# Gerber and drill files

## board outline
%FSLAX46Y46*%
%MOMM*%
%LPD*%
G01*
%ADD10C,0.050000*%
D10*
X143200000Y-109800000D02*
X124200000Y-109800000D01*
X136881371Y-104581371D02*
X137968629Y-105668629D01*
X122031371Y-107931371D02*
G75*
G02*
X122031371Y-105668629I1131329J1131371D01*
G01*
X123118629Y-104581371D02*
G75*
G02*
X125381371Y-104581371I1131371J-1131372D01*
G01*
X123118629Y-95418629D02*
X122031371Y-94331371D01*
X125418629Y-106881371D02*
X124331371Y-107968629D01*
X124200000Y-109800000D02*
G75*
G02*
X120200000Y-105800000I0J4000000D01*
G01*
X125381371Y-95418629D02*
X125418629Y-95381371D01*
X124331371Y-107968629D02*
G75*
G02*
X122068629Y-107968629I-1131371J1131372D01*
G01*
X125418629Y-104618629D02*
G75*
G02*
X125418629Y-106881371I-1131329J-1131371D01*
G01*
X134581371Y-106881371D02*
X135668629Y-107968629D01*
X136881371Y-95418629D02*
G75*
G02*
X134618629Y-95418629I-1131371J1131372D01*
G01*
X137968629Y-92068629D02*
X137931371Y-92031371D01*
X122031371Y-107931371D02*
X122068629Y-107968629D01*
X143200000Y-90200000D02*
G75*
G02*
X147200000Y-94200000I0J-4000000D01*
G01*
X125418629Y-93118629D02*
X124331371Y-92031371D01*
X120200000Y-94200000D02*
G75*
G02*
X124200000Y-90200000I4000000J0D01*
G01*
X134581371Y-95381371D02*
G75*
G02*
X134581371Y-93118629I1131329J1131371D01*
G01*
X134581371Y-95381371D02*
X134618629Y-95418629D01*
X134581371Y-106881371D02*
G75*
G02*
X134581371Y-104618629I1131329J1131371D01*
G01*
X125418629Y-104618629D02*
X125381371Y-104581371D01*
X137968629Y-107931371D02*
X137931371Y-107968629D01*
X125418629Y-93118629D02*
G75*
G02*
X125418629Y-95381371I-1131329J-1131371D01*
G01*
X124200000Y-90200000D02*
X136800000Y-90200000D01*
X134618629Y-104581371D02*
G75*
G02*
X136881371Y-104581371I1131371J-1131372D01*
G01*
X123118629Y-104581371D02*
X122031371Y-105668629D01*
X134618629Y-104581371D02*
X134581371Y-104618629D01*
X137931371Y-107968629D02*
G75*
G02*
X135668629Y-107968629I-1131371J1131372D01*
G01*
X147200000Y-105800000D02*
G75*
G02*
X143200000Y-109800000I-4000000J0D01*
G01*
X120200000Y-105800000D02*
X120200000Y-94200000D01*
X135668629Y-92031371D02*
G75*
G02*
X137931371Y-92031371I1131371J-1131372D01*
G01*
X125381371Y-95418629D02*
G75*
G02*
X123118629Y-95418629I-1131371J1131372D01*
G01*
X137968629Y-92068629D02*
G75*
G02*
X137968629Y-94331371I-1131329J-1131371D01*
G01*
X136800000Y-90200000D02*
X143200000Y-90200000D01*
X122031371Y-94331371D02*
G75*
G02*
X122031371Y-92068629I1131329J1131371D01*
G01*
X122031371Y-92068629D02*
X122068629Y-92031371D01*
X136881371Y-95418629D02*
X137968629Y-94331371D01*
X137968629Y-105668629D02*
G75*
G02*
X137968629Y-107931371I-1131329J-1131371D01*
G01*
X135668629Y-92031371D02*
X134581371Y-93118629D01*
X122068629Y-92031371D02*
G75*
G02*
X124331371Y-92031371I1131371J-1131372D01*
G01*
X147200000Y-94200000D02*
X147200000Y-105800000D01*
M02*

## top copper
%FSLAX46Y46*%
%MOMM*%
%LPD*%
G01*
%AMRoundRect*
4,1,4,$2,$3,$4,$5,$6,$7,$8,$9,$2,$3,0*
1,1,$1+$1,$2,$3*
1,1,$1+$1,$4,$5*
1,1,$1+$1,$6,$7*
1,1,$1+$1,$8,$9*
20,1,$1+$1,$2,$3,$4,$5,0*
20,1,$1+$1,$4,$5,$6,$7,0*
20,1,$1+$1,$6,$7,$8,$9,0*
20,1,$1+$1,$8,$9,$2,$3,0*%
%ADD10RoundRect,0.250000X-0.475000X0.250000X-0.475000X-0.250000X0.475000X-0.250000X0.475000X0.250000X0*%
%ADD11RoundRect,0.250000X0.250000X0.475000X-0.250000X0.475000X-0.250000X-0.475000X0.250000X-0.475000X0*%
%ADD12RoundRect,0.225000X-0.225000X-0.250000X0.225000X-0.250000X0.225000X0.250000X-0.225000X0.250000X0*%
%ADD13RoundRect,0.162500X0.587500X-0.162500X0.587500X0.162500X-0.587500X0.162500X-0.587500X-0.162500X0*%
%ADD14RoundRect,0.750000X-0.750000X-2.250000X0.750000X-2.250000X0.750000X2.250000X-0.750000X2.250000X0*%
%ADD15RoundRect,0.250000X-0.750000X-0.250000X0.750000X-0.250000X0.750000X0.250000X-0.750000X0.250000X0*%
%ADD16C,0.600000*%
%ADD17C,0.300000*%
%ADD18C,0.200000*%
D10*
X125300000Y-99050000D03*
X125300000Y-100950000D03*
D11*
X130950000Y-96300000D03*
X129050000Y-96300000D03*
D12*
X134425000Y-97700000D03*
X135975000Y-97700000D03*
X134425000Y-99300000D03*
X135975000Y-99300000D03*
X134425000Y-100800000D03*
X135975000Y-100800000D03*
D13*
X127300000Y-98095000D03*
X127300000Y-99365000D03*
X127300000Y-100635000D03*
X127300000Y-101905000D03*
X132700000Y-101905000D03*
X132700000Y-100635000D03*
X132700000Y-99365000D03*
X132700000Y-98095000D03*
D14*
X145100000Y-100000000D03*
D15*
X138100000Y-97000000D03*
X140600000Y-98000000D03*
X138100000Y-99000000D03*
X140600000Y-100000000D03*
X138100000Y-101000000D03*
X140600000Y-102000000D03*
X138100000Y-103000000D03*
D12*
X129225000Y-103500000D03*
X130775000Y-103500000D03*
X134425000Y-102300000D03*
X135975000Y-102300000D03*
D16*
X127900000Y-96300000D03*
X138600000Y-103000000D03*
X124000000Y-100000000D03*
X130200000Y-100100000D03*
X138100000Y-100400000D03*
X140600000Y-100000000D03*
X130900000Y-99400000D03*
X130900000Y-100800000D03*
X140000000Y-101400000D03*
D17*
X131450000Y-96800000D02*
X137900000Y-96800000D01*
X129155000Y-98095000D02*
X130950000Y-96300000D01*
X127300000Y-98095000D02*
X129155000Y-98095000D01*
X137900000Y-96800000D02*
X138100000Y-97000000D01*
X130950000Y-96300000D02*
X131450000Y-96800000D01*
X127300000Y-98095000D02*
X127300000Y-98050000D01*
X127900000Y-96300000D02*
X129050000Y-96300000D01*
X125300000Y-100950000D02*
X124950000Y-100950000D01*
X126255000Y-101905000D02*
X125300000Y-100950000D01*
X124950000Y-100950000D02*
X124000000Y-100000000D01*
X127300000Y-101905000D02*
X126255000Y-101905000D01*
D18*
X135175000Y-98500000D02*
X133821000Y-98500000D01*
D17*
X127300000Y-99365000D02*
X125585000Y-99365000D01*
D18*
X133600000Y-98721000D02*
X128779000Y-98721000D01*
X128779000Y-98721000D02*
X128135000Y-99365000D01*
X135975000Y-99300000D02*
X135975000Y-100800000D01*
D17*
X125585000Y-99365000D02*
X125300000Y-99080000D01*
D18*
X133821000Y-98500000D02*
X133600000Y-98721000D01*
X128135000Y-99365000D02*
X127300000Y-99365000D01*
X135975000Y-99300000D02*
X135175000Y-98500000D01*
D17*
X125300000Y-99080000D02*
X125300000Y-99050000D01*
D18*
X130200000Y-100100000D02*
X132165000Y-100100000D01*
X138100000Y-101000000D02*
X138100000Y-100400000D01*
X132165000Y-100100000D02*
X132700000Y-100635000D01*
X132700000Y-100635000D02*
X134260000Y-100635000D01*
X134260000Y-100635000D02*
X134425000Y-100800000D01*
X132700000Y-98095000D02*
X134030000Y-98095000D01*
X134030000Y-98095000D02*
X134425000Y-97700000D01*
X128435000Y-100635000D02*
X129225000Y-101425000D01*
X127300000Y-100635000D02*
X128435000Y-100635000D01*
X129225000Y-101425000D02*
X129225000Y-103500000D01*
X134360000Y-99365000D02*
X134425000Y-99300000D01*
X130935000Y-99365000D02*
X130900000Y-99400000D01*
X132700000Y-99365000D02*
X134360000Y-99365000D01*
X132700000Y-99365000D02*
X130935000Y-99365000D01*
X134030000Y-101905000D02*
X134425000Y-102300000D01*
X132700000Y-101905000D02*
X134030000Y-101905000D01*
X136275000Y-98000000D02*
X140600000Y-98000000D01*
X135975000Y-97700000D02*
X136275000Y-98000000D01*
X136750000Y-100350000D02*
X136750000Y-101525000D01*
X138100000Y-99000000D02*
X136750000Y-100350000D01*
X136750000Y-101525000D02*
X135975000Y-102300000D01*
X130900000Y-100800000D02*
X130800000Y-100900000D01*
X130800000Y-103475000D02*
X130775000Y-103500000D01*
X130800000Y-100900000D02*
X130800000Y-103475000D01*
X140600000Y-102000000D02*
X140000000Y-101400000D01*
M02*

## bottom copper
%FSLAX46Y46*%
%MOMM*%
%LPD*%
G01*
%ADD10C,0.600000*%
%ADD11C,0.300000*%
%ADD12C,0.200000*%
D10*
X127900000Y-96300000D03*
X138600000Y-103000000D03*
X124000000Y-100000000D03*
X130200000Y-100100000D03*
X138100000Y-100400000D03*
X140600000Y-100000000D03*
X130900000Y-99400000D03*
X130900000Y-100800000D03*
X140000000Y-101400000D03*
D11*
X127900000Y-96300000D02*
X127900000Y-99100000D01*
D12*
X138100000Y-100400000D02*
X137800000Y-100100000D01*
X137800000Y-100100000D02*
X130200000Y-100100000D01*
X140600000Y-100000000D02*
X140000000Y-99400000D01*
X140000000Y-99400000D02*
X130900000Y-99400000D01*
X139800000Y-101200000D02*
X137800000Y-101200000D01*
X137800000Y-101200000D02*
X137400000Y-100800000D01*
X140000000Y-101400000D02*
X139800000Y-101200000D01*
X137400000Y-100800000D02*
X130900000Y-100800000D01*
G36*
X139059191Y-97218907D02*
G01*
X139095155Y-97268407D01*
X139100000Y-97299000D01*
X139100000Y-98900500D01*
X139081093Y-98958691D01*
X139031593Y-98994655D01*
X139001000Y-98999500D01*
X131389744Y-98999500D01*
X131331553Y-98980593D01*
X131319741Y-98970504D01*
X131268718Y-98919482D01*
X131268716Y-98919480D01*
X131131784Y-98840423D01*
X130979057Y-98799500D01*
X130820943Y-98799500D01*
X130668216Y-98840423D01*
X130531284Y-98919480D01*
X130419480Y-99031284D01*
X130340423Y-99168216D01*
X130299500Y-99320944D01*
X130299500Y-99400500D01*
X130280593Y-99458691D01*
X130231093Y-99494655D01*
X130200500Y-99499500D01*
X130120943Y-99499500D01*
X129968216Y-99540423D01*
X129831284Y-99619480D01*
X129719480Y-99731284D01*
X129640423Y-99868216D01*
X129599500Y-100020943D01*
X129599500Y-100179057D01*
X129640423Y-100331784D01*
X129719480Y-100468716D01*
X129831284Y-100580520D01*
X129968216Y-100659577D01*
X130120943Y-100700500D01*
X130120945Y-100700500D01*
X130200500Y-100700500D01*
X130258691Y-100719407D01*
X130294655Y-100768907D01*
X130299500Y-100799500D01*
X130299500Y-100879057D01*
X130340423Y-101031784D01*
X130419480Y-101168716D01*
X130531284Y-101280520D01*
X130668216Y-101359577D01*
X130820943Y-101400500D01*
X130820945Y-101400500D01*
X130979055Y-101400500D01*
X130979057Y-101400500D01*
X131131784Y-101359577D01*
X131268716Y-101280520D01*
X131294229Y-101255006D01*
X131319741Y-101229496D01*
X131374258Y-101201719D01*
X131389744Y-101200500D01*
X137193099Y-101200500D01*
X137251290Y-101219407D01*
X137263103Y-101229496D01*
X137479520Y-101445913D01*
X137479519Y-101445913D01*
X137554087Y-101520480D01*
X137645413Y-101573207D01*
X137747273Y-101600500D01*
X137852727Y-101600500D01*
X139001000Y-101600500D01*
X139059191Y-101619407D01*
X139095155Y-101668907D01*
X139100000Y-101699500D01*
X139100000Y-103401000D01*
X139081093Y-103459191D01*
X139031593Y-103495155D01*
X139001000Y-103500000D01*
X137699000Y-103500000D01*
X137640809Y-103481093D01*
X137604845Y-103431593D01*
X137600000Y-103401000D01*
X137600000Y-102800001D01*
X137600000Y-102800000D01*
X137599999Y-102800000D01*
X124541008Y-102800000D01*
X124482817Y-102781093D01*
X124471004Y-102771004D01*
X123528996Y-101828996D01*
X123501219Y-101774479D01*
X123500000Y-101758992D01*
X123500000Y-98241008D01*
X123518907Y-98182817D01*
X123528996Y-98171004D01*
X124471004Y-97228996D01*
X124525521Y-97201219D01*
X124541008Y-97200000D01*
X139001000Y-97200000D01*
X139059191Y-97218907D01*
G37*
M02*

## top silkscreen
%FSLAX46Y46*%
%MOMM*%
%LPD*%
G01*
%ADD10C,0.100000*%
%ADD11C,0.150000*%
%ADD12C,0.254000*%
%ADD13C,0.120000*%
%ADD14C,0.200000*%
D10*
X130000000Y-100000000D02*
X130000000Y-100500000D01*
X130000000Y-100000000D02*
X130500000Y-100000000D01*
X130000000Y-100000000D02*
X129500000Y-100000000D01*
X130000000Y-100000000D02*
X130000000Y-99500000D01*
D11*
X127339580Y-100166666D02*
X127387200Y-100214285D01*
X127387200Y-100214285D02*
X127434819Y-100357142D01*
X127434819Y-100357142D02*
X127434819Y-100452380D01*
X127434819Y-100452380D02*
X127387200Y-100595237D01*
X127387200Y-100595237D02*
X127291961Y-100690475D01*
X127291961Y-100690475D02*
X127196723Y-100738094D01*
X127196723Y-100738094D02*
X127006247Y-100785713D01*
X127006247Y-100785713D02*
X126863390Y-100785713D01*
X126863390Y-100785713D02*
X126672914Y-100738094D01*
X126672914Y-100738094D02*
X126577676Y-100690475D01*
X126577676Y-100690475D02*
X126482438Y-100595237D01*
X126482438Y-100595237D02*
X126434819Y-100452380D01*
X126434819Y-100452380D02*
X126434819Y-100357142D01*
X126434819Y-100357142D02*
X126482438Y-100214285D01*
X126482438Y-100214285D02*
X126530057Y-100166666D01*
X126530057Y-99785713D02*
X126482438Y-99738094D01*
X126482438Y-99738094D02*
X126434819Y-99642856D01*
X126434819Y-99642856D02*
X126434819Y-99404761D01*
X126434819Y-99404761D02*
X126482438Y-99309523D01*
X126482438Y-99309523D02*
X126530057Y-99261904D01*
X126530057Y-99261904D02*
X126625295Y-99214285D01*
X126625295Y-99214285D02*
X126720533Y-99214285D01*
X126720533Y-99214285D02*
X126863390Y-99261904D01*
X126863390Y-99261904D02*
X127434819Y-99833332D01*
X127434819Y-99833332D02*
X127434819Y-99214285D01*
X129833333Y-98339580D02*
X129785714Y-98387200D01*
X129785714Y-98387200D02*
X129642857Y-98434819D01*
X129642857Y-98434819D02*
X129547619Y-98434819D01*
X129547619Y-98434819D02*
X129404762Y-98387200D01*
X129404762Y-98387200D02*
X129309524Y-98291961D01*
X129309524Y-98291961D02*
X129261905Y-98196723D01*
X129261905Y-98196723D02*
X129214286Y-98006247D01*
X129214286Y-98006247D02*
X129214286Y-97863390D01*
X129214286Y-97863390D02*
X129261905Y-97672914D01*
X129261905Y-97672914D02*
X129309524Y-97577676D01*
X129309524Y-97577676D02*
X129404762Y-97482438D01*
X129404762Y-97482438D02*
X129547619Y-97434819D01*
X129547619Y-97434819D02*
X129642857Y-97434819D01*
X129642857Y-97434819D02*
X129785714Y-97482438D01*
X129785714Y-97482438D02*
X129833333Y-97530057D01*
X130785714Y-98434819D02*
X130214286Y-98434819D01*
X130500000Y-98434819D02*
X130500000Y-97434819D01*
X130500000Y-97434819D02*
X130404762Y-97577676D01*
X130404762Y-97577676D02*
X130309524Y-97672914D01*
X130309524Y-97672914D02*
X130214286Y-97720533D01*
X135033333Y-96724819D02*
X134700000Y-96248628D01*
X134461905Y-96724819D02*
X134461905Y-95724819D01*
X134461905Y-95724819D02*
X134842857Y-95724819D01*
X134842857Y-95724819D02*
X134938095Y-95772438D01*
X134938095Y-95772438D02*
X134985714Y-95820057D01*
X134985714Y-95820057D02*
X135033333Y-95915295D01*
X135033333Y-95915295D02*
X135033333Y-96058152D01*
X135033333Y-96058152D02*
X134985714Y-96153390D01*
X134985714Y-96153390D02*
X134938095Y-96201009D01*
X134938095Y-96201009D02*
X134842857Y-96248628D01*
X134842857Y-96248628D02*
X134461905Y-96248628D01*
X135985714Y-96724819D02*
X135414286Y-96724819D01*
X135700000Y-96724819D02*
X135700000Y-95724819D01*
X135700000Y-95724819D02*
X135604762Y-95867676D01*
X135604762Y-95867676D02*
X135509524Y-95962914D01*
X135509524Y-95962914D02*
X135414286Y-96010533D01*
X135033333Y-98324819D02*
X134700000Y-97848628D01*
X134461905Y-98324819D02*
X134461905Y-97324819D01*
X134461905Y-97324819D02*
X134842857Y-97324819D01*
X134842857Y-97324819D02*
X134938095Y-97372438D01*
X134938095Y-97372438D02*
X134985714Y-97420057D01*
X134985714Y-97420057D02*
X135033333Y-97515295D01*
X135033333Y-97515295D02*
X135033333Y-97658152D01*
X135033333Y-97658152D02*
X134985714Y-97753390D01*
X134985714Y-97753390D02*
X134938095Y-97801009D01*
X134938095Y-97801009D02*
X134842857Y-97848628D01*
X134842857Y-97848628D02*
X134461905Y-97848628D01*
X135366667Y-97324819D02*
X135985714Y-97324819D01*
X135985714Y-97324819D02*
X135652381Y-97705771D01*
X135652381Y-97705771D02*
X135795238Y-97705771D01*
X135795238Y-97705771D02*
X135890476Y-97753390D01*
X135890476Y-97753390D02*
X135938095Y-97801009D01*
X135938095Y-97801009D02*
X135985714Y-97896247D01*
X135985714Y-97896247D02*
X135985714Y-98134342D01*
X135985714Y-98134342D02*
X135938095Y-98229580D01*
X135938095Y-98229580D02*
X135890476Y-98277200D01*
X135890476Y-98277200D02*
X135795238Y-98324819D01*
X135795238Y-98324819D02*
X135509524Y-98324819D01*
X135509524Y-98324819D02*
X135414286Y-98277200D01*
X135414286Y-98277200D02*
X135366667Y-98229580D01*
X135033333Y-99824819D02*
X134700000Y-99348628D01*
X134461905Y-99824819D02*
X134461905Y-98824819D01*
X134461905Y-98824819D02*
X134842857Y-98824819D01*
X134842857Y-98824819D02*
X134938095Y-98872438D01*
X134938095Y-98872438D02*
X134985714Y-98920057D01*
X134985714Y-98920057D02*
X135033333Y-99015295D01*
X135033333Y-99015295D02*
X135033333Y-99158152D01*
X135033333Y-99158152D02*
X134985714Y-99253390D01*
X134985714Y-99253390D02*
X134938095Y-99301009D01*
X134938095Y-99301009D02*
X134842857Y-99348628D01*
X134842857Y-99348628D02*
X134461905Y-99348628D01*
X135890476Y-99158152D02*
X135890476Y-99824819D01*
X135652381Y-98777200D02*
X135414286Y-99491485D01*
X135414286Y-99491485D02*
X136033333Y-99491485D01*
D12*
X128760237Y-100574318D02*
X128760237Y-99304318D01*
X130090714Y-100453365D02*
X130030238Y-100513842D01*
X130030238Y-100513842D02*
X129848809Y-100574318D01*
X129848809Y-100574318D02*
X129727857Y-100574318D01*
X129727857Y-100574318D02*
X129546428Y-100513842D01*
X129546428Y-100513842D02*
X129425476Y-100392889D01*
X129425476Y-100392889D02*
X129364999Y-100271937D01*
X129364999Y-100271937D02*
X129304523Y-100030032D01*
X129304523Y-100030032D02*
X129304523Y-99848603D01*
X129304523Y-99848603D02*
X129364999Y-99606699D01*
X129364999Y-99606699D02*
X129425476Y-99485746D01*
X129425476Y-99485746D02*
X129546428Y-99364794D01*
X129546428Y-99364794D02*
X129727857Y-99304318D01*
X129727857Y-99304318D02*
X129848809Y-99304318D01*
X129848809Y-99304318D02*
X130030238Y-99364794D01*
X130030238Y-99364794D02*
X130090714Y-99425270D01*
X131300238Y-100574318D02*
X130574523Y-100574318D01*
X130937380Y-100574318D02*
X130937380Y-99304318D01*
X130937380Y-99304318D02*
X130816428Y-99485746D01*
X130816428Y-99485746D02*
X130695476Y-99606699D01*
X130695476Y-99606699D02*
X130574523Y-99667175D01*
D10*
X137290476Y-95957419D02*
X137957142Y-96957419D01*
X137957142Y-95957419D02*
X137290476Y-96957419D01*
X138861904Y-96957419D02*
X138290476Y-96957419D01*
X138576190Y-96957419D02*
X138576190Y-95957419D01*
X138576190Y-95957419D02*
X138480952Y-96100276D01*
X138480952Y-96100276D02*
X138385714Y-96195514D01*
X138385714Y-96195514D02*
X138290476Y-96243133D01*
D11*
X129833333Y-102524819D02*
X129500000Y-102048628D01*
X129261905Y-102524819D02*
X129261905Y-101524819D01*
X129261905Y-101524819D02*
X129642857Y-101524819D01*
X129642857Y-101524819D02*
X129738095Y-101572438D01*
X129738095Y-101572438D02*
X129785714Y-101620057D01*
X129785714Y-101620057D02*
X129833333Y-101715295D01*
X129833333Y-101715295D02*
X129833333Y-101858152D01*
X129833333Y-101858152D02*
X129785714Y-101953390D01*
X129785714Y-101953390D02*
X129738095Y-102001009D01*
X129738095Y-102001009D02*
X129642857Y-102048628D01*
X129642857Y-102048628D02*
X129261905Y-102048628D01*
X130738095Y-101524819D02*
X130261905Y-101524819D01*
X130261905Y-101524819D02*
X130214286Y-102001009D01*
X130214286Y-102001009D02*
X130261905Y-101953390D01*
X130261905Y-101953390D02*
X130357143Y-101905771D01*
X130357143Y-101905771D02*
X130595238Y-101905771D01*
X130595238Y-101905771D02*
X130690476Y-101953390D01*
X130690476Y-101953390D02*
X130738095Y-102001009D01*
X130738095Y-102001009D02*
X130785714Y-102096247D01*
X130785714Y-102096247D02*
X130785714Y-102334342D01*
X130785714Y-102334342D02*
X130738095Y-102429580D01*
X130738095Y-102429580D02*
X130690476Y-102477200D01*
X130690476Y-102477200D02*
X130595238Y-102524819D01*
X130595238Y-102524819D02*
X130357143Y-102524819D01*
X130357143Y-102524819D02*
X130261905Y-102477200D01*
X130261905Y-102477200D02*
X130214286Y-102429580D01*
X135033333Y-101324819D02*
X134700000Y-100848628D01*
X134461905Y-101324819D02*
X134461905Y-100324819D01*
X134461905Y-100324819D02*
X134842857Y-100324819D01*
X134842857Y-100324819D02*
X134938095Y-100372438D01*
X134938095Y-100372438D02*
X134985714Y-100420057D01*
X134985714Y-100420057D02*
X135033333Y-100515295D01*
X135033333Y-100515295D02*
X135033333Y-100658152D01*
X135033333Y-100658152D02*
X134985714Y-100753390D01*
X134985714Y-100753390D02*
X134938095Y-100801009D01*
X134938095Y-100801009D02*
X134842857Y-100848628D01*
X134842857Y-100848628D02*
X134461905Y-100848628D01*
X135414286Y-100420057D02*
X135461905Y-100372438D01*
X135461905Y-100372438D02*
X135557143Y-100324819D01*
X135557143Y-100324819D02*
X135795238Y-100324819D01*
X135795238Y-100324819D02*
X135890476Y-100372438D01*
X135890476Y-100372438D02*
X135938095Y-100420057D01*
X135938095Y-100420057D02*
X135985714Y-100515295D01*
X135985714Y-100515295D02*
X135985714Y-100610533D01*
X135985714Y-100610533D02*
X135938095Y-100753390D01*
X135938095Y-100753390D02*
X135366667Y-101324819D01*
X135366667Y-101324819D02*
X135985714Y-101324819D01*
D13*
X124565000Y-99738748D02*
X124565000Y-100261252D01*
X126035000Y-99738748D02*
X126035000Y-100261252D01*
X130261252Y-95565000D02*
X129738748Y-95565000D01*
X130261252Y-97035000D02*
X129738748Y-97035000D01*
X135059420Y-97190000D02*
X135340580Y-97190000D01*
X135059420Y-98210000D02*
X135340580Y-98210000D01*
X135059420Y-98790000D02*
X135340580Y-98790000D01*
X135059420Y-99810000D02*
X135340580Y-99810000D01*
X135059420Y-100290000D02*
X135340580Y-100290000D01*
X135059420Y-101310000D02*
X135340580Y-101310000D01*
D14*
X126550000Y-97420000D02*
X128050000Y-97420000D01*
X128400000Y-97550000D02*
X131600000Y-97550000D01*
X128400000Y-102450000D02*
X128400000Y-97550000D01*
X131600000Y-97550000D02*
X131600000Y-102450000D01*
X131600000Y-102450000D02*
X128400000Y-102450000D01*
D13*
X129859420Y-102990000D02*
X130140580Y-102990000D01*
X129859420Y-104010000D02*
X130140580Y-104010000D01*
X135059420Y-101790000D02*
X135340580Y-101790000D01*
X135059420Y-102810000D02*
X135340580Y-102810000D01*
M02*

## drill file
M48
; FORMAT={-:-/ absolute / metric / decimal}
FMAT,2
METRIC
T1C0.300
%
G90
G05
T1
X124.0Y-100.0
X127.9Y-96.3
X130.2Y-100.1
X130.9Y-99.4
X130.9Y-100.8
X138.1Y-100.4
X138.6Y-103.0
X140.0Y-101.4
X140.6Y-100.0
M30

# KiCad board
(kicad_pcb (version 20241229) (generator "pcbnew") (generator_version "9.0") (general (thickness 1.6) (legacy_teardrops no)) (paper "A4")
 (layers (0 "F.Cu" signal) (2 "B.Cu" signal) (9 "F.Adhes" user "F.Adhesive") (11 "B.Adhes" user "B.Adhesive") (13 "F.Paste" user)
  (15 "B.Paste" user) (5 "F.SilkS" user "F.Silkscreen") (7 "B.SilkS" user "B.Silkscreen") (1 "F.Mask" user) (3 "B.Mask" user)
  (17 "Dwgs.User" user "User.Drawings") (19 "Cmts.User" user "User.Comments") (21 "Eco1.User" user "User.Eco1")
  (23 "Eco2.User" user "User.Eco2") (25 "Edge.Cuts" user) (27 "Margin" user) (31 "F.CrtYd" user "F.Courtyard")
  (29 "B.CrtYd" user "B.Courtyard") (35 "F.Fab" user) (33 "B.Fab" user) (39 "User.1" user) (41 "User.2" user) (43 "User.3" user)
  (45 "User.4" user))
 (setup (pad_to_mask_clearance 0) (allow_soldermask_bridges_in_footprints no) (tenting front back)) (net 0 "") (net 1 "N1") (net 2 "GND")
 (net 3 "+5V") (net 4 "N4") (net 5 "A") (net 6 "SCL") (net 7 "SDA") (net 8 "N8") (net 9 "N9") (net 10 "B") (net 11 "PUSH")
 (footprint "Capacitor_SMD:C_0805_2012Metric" (layer "F.Cu") (at 125.3 100 -90)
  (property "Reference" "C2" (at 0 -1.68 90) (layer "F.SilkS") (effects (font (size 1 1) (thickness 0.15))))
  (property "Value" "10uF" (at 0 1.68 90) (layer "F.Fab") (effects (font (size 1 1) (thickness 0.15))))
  (fp_line (start -0.261252 0.735) (end 0.261252 0.735) (stroke (width 0.12) (type solid)) (layer "F.SilkS"))
  (fp_line (start -0.261252 -0.735) (end 0.261252 -0.735) (stroke (width 0.12) (type solid)) (layer "F.SilkS"))
  (pad "1" smd roundrect (at -0.95 0 270) (size 1 1.45) (layers "F.Cu" "F.Mask" "F.Paste") (roundrect_rratio 0.25) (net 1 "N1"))
  (pad "2" smd roundrect (at 0.95 0 270) (size 1 1.45) (layers "F.Cu" "F.Mask" "F.Paste") (roundrect_rratio 0.25) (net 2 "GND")))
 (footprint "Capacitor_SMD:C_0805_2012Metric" (layer "F.Cu") (at 130 96.3 180)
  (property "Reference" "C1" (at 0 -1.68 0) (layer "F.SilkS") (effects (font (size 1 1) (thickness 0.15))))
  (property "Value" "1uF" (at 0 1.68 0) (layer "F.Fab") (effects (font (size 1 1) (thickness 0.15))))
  (fp_line (start -0.261252 0.735) (end 0.261252 0.735) (stroke (width 0.12) (type solid)) (layer "F.SilkS"))
  (fp_line (start -0.261252 -0.735) (end 0.261252 -0.735) (stroke (width 0.12) (type solid)) (layer "F.SilkS"))
  (pad "1" smd roundrect (at -0.95 0 180) (size 1 1.45) (layers "F.Cu" "F.Mask" "F.Paste") (roundrect_rratio 0.25) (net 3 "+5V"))
  (pad "2" smd roundrect (at 0.95 0 180) (size 1 1.45) (layers "F.Cu" "F.Mask" "F.Paste") (roundrect_rratio 0.25) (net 2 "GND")))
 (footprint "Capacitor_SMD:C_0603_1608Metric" (layer "F.Cu") (at 135.2 97.7)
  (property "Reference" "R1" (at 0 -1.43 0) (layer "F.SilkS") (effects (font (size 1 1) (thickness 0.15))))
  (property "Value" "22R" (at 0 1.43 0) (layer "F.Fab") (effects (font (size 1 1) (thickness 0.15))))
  (fp_line (start -0.14058 -0.51) (end 0.14058 -0.51) (stroke (width 0.12) (type solid)) (layer "F.SilkS"))
  (fp_line (start -0.14058 0.51) (end 0.14058 0.51) (stroke (width 0.12) (type solid)) (layer "F.SilkS"))
  (pad "1" smd roundrect (at -0.775 0) (size 0.9 0.95) (layers "F.Cu" "F.Mask" "F.Paste") (roundrect_rratio 0.25) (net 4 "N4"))
  (pad "2" smd roundrect (at 0.775 0) (size 0.9 0.95) (layers "F.Cu" "F.Mask" "F.Paste") (roundrect_rratio 0.25) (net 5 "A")))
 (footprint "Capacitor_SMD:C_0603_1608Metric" (layer "F.Cu") (at 135.2 99.3)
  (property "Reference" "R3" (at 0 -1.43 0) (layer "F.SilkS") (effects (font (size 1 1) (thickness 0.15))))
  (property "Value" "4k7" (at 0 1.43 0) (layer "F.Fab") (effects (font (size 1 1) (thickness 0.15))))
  (fp_line (start -0.14058 -0.51) (end 0.14058 -0.51) (stroke (width 0.12) (type solid)) (layer "F.SilkS"))
  (fp_line (start -0.14058 0.51) (end 0.14058 0.51) (stroke (width 0.12) (type solid)) (layer "F.SilkS"))
  (pad "1" smd roundrect (at -0.775 0) (size 0.9 0.95) (layers "F.Cu" "F.Mask" "F.Paste") (roundrect_rratio 0.25) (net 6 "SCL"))
  (pad "2" smd roundrect (at 0.775 0) (size 0.9 0.95) (layers "F.Cu" "F.Mask" "F.Paste") (roundrect_rratio 0.25) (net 1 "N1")))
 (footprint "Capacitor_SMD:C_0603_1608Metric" (layer "F.Cu") (at 135.2 100.8)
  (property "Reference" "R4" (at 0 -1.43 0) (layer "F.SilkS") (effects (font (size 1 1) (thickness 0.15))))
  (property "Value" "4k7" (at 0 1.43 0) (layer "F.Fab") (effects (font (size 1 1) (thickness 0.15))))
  (fp_line (start -0.14058 -0.51) (end 0.14058 -0.51) (stroke (width 0.12) (type solid)) (layer "F.SilkS"))
  (fp_line (start -0.14058 0.51) (end 0.14058 0.51) (stroke (width 0.12) (type solid)) (layer "F.SilkS"))
  (pad "1" smd roundrect (at -0.775 0) (size 0.9 0.95) (layers "F.Cu" "F.Mask" "F.Paste") (roundrect_rratio 0.25) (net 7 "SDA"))
  (pad "2" smd roundrect (at 0.775 0) (size 0.9 0.95) (layers "F.Cu" "F.Mask" "F.Paste") (roundrect_rratio 0.25) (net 1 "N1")))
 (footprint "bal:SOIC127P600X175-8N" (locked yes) (layer "F.Cu") (at 130 100)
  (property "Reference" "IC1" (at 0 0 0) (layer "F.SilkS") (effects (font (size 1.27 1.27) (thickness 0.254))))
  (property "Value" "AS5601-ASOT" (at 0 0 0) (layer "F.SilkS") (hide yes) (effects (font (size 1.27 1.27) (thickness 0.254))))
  (fp_line (start -3.45 -2.58) (end -1.95 -2.58) (stroke (width 0.2) (type solid)) (layer "F.SilkS"))
  (fp_line (start -1.6 -2.45) (end 1.6 -2.45) (stroke (width 0.2) (type solid)) (layer "F.SilkS"))
  (fp_line (start -1.6 2.45) (end -1.6 -2.45) (stroke (width 0.2) (type solid)) (layer "F.SilkS"))
  (fp_line (start 1.6 -2.45) (end 1.6 2.45) (stroke (width 0.2) (type solid)) (layer "F.SilkS"))
  (fp_line (start 1.6 2.45) (end -1.6 2.45) (stroke (width 0.2) (type solid)) (layer "F.SilkS"))
  (pad "1" smd roundrect (at -2.7 -1.905 90) (size 0.65 1.5) (layers "F.Cu" "F.Mask" "F.Paste") (roundrect_rratio 0.25) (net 3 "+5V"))
  (pad "2" smd roundrect (at -2.7 -0.635 90) (size 0.65 1.5) (layers "F.Cu" "F.Mask" "F.Paste") (roundrect_rratio 0.25) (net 1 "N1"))
  (pad "3" smd roundrect (at -2.7 0.635 90) (size 0.65 1.5) (layers "F.Cu" "F.Mask" "F.Paste") (roundrect_rratio 0.25) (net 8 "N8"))
  (pad "4" smd roundrect (at -2.7 1.905 90) (size 0.65 1.5) (layers "F.Cu" "F.Mask" "F.Paste") (roundrect_rratio 0.25) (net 2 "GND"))
  (pad "5" smd roundrect (at 2.7 1.905 90) (size 0.65 1.5) (layers "F.Cu" "F.Mask" "F.Paste") (roundrect_rratio 0.25) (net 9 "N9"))
  (pad "6" smd roundrect (at 2.7 0.635 90) (size 0.65 1.5) (layers "F.Cu" "F.Mask" "F.Paste") (roundrect_rratio 0.25) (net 7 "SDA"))
  (pad "7" smd roundrect (at 2.7 -0.635 90) (size 0.65 1.5) (layers "F.Cu" "F.Mask" "F.Paste") (roundrect_rratio 0.25) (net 6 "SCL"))
  (pad "8" smd roundrect (at 2.7 -1.905 90) (size 0.65 1.5) (layers "F.Cu" "F.Mask" "F.Paste") (roundrect_rratio 0.25) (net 4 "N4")))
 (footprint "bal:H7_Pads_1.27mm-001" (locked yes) (layer "F.Cu") (at 138.1 97)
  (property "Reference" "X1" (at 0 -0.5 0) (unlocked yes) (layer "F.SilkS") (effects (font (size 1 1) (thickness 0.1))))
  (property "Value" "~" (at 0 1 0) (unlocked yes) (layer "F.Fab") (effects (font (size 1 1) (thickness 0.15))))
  (pad "" smd roundrect (at 7 3) (size 3 6) (layers "F.Cu" "F.Mask" "F.Paste") (roundrect_rratio 0.25) (thermal_bridge_angle 45))
  (pad "1" smd roundrect (at 0 0) (size 2 1) (layers "F.Cu" "F.Mask" "F.Paste") (roundrect_rratio 0.25) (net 3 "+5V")
   (thermal_bridge_angle 45))
  (pad "2" smd roundrect (at 2.5 1) (size 2 1) (layers "F.Cu" "F.Mask" "F.Paste") (roundrect_rratio 0.25) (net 5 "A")
   (thermal_bridge_angle 45))
  (pad "3" smd roundrect (at 0 2) (size 2 1) (layers "F.Cu" "F.Mask" "F.Paste") (roundrect_rratio 0.25) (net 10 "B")
   (thermal_bridge_angle 45))
  (pad "4" smd roundrect (at 2.5 3) (size 2 1) (layers "F.Cu" "F.Mask" "F.Paste") (roundrect_rratio 0.25) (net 6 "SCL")
   (thermal_bridge_angle 45))
  (pad "5" smd roundrect (at 0 4) (size 2 1) (layers "F.Cu" "F.Mask" "F.Paste") (roundrect_rratio 0.25) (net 7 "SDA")
   (thermal_bridge_angle 45))
  (pad "6" smd roundrect (at 2.5 5) (size 2 1) (layers "F.Cu" "F.Mask" "F.Paste") (roundrect_rratio 0.25) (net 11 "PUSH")
   (thermal_bridge_angle 45))
  (pad "7" smd roundrect (at 0 6) (size 2 1) (layers "F.Cu" "F.Mask" "F.Paste") (roundrect_rratio 0.25) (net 2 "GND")
   (thermal_bridge_angle 45)))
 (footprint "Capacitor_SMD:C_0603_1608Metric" (layer "F.Cu") (at 130 103.5)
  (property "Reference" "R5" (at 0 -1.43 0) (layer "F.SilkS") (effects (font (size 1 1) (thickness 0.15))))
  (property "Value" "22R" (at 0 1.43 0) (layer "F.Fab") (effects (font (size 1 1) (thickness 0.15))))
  (fp_line (start -0.14058 -0.51) (end 0.14058 -0.51) (stroke (width 0.12) (type solid)) (layer "F.SilkS"))
  (fp_line (start -0.14058 0.51) (end 0.14058 0.51) (stroke (width 0.12) (type solid)) (layer "F.SilkS"))
  (pad "1" smd roundrect (at -0.775 0) (size 0.9 0.95) (layers "F.Cu" "F.Mask" "F.Paste") (roundrect_rratio 0.25) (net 8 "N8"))
  (pad "2" smd roundrect (at 0.775 0) (size 0.9 0.95) (layers "F.Cu" "F.Mask" "F.Paste") (roundrect_rratio 0.25) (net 11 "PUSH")))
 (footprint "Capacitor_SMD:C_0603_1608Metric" (layer "F.Cu") (at 135.2 102.3)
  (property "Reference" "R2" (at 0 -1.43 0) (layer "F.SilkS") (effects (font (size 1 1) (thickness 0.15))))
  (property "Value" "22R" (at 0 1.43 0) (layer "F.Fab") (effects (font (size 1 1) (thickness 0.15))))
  (fp_line (start -0.14058 -0.51) (end 0.14058 -0.51) (stroke (width 0.12) (type solid)) (layer "F.SilkS"))
  (fp_line (start -0.14058 0.51) (end 0.14058 0.51) (stroke (width 0.12) (type solid)) (layer "F.SilkS"))
  (pad "1" smd roundrect (at -0.775 0) (size 0.9 0.95) (layers "F.Cu" "F.Mask" "F.Paste") (roundrect_rratio 0.25) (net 9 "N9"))
  (pad "2" smd roundrect (at 0.775 0) (size 0.9 0.95) (layers "F.Cu" "F.Mask" "F.Paste") (roundrect_rratio 0.25) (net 10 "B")))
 (gr_line (start 130 100) (end 130 100.5) (stroke (width 0.1) (type default)) (layer "F.SilkS"))
 (gr_line (start 130 100) (end 130.5 100) (stroke (width 0.1) (type default)) (layer "F.SilkS"))
 (gr_line (start 130 100) (end 129.5 100) (stroke (width 0.1) (type default)) (layer "F.SilkS"))
 (gr_line (start 130 100) (end 130 99.5) (stroke (width 0.1) (type default)) (layer "F.SilkS"))
 (gr_line (start 143.2 109.8) (end 124.2 109.8) (stroke (width 0.05) (type default)) (layer "Edge.Cuts"))
 (gr_line (start 136.881371 104.581371) (end 137.968629 105.668629) (stroke (width 0.05) (type default)) (layer "Edge.Cuts"))
 (gr_arc (start 122.031371 107.931371) (mid 121.562729 106.8) (end 122.031371 105.668629) (stroke (width 0.05) (type default))
  (layer "Edge.Cuts"))
 (gr_arc (start 123.118629 104.581371) (mid 124.25 104.112742) (end 125.381371 104.581371) (stroke (width 0.05) (type default))
  (layer "Edge.Cuts"))
 (gr_line (start 123.118629 95.418629) (end 122.031371 94.331371) (stroke (width 0.05) (type default)) (layer "Edge.Cuts"))
 (gr_line (start 125.418629 106.881371) (end 124.331371 107.968629) (stroke (width 0.05) (type default)) (layer "Edge.Cuts"))
 (gr_arc (start 124.2 109.8) (mid 121.371573 108.628427) (end 120.2 105.8) (stroke (width 0.05) (type default)) (layer "Edge.Cuts"))
 (gr_line (start 125.381371 95.418629) (end 125.418629 95.381371) (stroke (width 0.05) (type default)) (layer "Edge.Cuts"))
 (gr_arc (start 124.331371 107.968629) (mid 123.2 108.437258) (end 122.068629 107.968629) (stroke (width 0.05) (type default))
  (layer "Edge.Cuts"))
 (gr_arc (start 125.418629 104.618629) (mid 125.887258 105.75) (end 125.418629 106.881371) (stroke (width 0.05) (type default))
  (layer "Edge.Cuts"))
 (gr_line (start 134.581371 106.881371) (end 135.668629 107.968629) (stroke (width 0.05) (type default)) (layer "Edge.Cuts"))
 (gr_arc (start 136.881371 95.418629) (mid 135.75 95.887258) (end 134.618629 95.418629) (stroke (width 0.05) (type default))
  (layer "Edge.Cuts"))
 (gr_line (start 137.968629 92.068629) (end 137.931371 92.031371) (stroke (width 0.05) (type default)) (layer "Edge.Cuts"))
 (gr_line (start 122.031371 107.931371) (end 122.068629 107.968629) (stroke (width 0.05) (type default)) (layer "Edge.Cuts"))
 (gr_arc (start 143.2 90.2) (mid 146.028427 91.371573) (end 147.2 94.2) (stroke (width 0.05) (type default)) (layer "Edge.Cuts"))
 (gr_line (start 125.418629 93.118629) (end 124.331371 92.031371) (stroke (width 0.05) (type default)) (layer "Edge.Cuts"))
 (gr_arc (start 120.2 94.2) (mid 121.371573 91.371573) (end 124.2 90.2) (stroke (width 0.05) (type default)) (layer "Edge.Cuts"))
 (gr_arc (start 134.581371 95.381371) (mid 134.112729 94.25) (end 134.581371 93.118629) (stroke (width 0.05) (type default))
  (layer "Edge.Cuts"))
 (gr_line (start 134.581371 95.381371) (end 134.618629 95.418629) (stroke (width 0.05) (type default)) (layer "Edge.Cuts"))
 (gr_arc (start 134.581371 106.881371) (mid 134.112729 105.75) (end 134.581371 104.618629) (stroke (width 0.05) (type default))
  (layer "Edge.Cuts"))
 (gr_line (start 125.418629 104.618629) (end 125.381371 104.581371) (stroke (width 0.05) (type default)) (layer "Edge.Cuts"))
 (gr_line (start 137.968629 107.931371) (end 137.931371 107.968629) (stroke (width 0.05) (type default)) (layer "Edge.Cuts"))
 (gr_arc (start 125.418629 93.118629) (mid 125.887258 94.25) (end 125.418629 95.381371) (stroke (width 0.05) (type default))
  (layer "Edge.Cuts"))
 (gr_line (start 124.2 90.2) (end 136.8 90.2) (stroke (width 0.05) (type default)) (layer "Edge.Cuts"))
 (gr_arc (start 134.618629 104.581371) (mid 135.75 104.112742) (end 136.881371 104.581371) (stroke (width 0.05) (type default))
  (layer "Edge.Cuts"))
 (gr_line (start 123.118629 104.581371) (end 122.031371 105.668629) (stroke (width 0.05) (type default)) (layer "Edge.Cuts"))
 (gr_line (start 134.618629 104.581371) (end 134.581371 104.618629) (stroke (width 0.05) (type default)) (layer "Edge.Cuts"))
 (gr_arc (start 137.931371 107.968629) (mid 136.8 108.437258) (end 135.668629 107.968629) (stroke (width 0.05) (type default))
  (layer "Edge.Cuts"))
 (gr_arc (start 147.2 105.8) (mid 146.028427 108.628427) (end 143.2 109.8) (stroke (width 0.05) (type default)) (layer "Edge.Cuts"))
 (gr_line (start 120.2 105.8) (end 120.2 94.2) (stroke (width 0.05) (type default)) (layer "Edge.Cuts"))
 (gr_arc (start 135.668629 92.031371) (mid 136.8 91.562742) (end 137.931371 92.031371) (stroke (width 0.05) (type default))
  (layer "Edge.Cuts"))
 (gr_arc (start 125.381371 95.418629) (mid 124.25 95.887258) (end 123.118629 95.418629) (stroke (width 0.05) (type default))
  (layer "Edge.Cuts"))
 (gr_arc (start 137.968629 92.068629) (mid 138.437258 93.2) (end 137.968629 94.331371) (stroke (width 0.05) (type default))
  (layer "Edge.Cuts"))
 (gr_line (start 136.8 90.2) (end 143.2 90.2) (stroke (width 0.05) (type default)) (layer "Edge.Cuts"))
 (gr_arc (start 122.031371 94.331371) (mid 121.562729 93.2) (end 122.031371 92.068629) (stroke (width 0.05) (type default))
  (layer "Edge.Cuts"))
 (gr_line (start 122.031371 92.068629) (end 122.068629 92.031371) (stroke (width 0.05) (type default)) (layer "Edge.Cuts"))
 (gr_line (start 136.881371 95.418629) (end 137.968629 94.331371) (stroke (width 0.05) (type default)) (layer "Edge.Cuts"))
 (gr_arc (start 137.968629 105.668629) (mid 138.437271 106.8) (end 137.968629 107.931371) (stroke (width 0.05) (type default))
  (layer "Edge.Cuts"))
 (gr_line (start 135.668629 92.031371) (end 134.581371 93.118629) (stroke (width 0.05) (type default)) (layer "Edge.Cuts"))
 (gr_arc (start 122.068629 92.031371) (mid 123.2 91.562742) (end 124.331371 92.031371) (stroke (width 0.05) (type default))
  (layer "Edge.Cuts"))
 (gr_line (start 147.2 94.2) (end 147.2 105.8) (stroke (width 0.05) (type default)) (layer "Edge.Cuts"))
 (segment (start 131.45 96.8) (end 137.9 96.8) (width 0.3) (layer "F.Cu") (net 3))
 (segment (start 129.155 98.095) (end 130.95 96.3) (width 0.3) (layer "F.Cu") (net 3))
 (segment (start 127.3 98.095) (end 129.155 98.095) (width 0.3) (layer "F.Cu") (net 3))
 (segment (start 137.9 96.8) (end 138.1 97) (width 0.3) (layer "F.Cu") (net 3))
 (segment (start 130.95 96.3) (end 131.45 96.8) (width 0.3) (layer "F.Cu") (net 3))
 (segment (start 127.3 98.095) (end 127.3 98.05) (width 0.3) (layer "F.Cu") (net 3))
 (segment (start 127.9 96.3) (end 129.05 96.3) (width 0.3) (layer "F.Cu") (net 2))
 (segment (start 125.3 100.95) (end 124.95 100.95) (width 0.3) (layer "F.Cu") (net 2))
 (segment (start 126.255 101.905) (end 125.3 100.95) (width 0.3) (layer "F.Cu") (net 2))
 (segment (start 124.95 100.95) (end 124 100) (width 0.3) (layer "F.Cu") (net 2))
 (segment (start 127.3 101.905) (end 126.255 101.905) (width 0.3) (layer "F.Cu") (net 2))
 (via (at 127.9 96.3) (size 0.6) (drill 0.3) (layers "F.Cu" "B.Cu") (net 2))
 (via (at 138.6 103) (size 0.6) (drill 0.3) (layers "F.Cu" "B.Cu") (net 2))
 (via (at 124 100) (size 0.6) (drill 0.3) (layers "F.Cu" "B.Cu") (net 2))
 (segment (start 127.9 96.3) (end 127.9 99.1) (width 0.3) (layer "B.Cu") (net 2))
 (segment (start 135.175 98.5) (end 133.821 98.5) (width 0.2) (layer "F.Cu") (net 1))
 (segment (start 127.3 99.365) (end 125.585 99.365) (width 0.3) (layer "F.Cu") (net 1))
 (segment (start 133.6 98.721) (end 128.779 98.721) (width 0.2) (layer "F.Cu") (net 1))
 (segment (start 128.779 98.721) (end 128.135 99.365) (width 0.2) (layer "F.Cu") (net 1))
 (segment (start 135.975 99.3) (end 135.975 100.8) (width 0.2) (layer "F.Cu") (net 1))
 (segment (start 125.585 99.365) (end 125.3 99.08) (width 0.3) (layer "F.Cu") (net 1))
 (segment (start 133.821 98.5) (end 133.6 98.721) (width 0.2) (layer "F.Cu") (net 1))
 (segment (start 128.135 99.365) (end 127.3 99.365) (width 0.2) (layer "F.Cu") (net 1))
 (segment (start 135.975 99.3) (end 135.175 98.5) (width 0.2) (layer "F.Cu") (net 1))
 (segment (start 125.3 99.08) (end 125.3 99.05) (width 0.3) (layer "F.Cu") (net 1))
 (segment (start 130.2 100.1) (end 132.165 100.1) (width 0.2) (layer "F.Cu") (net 7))
 (segment (start 138.1 101) (end 138.1 100.4) (width 0.2) (layer "F.Cu") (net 7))
 (segment (start 132.165 100.1) (end 132.7 100.635) (width 0.2) (layer "F.Cu") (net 7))
 (segment (start 132.7 100.635) (end 134.26 100.635) (width 0.2) (layer "F.Cu") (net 7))
 (segment (start 134.26 100.635) (end 134.425 100.8) (width 0.2) (layer "F.Cu") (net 7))
 (via (at 130.2 100.1) (size 0.6) (drill 0.3) (layers "F.Cu" "B.Cu") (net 7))
 (via (at 138.1 100.4) (size 0.6) (drill 0.3) (layers "F.Cu" "B.Cu") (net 7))
 (segment (start 138.1 100.4) (end 137.8 100.1) (width 0.2) (layer "B.Cu") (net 7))
 (segment (start 137.8 100.1) (end 130.2 100.1) (width 0.2) (layer "B.Cu") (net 7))
 (segment (start 132.7 98.095) (end 134.03 98.095) (width 0.2) (layer "F.Cu") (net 4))
 (segment (start 134.03 98.095) (end 134.425 97.7) (width 0.2) (layer "F.Cu") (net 4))
 (segment (start 128.435 100.635) (end 129.225 101.425) (width 0.2) (layer "F.Cu") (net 8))
 (segment (start 127.3 100.635) (end 128.435 100.635) (width 0.2) (layer "F.Cu") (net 8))
 (segment (start 129.225 101.425) (end 129.225 103.5) (width 0.2) (layer "F.Cu") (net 8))
 (segment (start 134.36 99.365) (end 134.425 99.3) (width 0.2) (layer "F.Cu") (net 6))
 (segment (start 130.935 99.365) (end 130.9 99.4) (width 0.2) (layer "F.Cu") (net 6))
 (segment (start 132.7 99.365) (end 134.36 99.365) (width 0.2) (layer "F.Cu") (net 6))
 (segment (start 132.7 99.365) (end 130.935 99.365) (width 0.2) (layer "F.Cu") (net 6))
 (via (at 140.6 100) (size 0.6) (drill 0.3) (layers "F.Cu" "B.Cu") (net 6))
 (via (at 130.9 99.4) (size 0.6) (drill 0.3) (layers "F.Cu" "B.Cu") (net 6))
 (segment (start 140.6 100) (end 140 99.4) (width 0.2) (layer "B.Cu") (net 6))
 (segment (start 140 99.4) (end 130.9 99.4) (width 0.2) (layer "B.Cu") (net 6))
 (segment (start 134.03 101.905) (end 134.425 102.3) (width 0.2) (layer "F.Cu") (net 9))
 (segment (start 132.7 101.905) (end 134.03 101.905) (width 0.2) (layer "F.Cu") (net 9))
 (segment (start 136.275 98) (end 140.6 98) (width 0.2) (layer "F.Cu") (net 5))
 (segment (start 135.975 97.7) (end 136.275 98) (width 0.2) (layer "F.Cu") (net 5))
 (segment (start 136.75 100.35) (end 136.75 101.525) (width 0.2) (layer "F.Cu") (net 10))
 (segment (start 138.1 99) (end 136.75 100.35) (width 0.2) (layer "F.Cu") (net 10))
 (segment (start 136.75 101.525) (end 135.975 102.3) (width 0.2) (layer "F.Cu") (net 10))
 (segment (start 130.9 100.8) (end 130.8 100.9) (width 0.2) (layer "F.Cu") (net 11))
 (segment (start 130.8 103.475) (end 130.775 103.5) (width 0.2) (layer "F.Cu") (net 11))
 (segment (start 130.8 100.9) (end 130.8 103.475) (width 0.2) (layer "F.Cu") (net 11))
 (segment (start 140.6 102) (end 140 101.4) (width 0.2) (layer "F.Cu") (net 11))
 (via (at 130.9 100.8) (size 0.6) (drill 0.3) (layers "F.Cu" "B.Cu") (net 11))
 (via (at 140 101.4) (size 0.6) (drill 0.3) (layers "F.Cu" "B.Cu") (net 11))
 (segment (start 139.8 101.2) (end 137.8 101.2) (width 0.2) (layer "B.Cu") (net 11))
 (segment (start 137.8 101.2) (end 137.4 100.8) (width 0.2) (layer "B.Cu") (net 11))
 (segment (start 140 101.4) (end 139.8 101.2) (width 0.2) (layer "B.Cu") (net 11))
 (segment (start 137.4 100.8) (end 130.9 100.8) (width 0.2) (layer "B.Cu") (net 11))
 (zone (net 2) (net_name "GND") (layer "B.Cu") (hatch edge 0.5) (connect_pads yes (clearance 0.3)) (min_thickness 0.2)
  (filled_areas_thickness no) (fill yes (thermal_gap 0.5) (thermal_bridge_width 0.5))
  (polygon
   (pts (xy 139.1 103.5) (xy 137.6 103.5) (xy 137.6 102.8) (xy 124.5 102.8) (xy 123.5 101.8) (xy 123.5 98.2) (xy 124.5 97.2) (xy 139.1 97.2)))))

